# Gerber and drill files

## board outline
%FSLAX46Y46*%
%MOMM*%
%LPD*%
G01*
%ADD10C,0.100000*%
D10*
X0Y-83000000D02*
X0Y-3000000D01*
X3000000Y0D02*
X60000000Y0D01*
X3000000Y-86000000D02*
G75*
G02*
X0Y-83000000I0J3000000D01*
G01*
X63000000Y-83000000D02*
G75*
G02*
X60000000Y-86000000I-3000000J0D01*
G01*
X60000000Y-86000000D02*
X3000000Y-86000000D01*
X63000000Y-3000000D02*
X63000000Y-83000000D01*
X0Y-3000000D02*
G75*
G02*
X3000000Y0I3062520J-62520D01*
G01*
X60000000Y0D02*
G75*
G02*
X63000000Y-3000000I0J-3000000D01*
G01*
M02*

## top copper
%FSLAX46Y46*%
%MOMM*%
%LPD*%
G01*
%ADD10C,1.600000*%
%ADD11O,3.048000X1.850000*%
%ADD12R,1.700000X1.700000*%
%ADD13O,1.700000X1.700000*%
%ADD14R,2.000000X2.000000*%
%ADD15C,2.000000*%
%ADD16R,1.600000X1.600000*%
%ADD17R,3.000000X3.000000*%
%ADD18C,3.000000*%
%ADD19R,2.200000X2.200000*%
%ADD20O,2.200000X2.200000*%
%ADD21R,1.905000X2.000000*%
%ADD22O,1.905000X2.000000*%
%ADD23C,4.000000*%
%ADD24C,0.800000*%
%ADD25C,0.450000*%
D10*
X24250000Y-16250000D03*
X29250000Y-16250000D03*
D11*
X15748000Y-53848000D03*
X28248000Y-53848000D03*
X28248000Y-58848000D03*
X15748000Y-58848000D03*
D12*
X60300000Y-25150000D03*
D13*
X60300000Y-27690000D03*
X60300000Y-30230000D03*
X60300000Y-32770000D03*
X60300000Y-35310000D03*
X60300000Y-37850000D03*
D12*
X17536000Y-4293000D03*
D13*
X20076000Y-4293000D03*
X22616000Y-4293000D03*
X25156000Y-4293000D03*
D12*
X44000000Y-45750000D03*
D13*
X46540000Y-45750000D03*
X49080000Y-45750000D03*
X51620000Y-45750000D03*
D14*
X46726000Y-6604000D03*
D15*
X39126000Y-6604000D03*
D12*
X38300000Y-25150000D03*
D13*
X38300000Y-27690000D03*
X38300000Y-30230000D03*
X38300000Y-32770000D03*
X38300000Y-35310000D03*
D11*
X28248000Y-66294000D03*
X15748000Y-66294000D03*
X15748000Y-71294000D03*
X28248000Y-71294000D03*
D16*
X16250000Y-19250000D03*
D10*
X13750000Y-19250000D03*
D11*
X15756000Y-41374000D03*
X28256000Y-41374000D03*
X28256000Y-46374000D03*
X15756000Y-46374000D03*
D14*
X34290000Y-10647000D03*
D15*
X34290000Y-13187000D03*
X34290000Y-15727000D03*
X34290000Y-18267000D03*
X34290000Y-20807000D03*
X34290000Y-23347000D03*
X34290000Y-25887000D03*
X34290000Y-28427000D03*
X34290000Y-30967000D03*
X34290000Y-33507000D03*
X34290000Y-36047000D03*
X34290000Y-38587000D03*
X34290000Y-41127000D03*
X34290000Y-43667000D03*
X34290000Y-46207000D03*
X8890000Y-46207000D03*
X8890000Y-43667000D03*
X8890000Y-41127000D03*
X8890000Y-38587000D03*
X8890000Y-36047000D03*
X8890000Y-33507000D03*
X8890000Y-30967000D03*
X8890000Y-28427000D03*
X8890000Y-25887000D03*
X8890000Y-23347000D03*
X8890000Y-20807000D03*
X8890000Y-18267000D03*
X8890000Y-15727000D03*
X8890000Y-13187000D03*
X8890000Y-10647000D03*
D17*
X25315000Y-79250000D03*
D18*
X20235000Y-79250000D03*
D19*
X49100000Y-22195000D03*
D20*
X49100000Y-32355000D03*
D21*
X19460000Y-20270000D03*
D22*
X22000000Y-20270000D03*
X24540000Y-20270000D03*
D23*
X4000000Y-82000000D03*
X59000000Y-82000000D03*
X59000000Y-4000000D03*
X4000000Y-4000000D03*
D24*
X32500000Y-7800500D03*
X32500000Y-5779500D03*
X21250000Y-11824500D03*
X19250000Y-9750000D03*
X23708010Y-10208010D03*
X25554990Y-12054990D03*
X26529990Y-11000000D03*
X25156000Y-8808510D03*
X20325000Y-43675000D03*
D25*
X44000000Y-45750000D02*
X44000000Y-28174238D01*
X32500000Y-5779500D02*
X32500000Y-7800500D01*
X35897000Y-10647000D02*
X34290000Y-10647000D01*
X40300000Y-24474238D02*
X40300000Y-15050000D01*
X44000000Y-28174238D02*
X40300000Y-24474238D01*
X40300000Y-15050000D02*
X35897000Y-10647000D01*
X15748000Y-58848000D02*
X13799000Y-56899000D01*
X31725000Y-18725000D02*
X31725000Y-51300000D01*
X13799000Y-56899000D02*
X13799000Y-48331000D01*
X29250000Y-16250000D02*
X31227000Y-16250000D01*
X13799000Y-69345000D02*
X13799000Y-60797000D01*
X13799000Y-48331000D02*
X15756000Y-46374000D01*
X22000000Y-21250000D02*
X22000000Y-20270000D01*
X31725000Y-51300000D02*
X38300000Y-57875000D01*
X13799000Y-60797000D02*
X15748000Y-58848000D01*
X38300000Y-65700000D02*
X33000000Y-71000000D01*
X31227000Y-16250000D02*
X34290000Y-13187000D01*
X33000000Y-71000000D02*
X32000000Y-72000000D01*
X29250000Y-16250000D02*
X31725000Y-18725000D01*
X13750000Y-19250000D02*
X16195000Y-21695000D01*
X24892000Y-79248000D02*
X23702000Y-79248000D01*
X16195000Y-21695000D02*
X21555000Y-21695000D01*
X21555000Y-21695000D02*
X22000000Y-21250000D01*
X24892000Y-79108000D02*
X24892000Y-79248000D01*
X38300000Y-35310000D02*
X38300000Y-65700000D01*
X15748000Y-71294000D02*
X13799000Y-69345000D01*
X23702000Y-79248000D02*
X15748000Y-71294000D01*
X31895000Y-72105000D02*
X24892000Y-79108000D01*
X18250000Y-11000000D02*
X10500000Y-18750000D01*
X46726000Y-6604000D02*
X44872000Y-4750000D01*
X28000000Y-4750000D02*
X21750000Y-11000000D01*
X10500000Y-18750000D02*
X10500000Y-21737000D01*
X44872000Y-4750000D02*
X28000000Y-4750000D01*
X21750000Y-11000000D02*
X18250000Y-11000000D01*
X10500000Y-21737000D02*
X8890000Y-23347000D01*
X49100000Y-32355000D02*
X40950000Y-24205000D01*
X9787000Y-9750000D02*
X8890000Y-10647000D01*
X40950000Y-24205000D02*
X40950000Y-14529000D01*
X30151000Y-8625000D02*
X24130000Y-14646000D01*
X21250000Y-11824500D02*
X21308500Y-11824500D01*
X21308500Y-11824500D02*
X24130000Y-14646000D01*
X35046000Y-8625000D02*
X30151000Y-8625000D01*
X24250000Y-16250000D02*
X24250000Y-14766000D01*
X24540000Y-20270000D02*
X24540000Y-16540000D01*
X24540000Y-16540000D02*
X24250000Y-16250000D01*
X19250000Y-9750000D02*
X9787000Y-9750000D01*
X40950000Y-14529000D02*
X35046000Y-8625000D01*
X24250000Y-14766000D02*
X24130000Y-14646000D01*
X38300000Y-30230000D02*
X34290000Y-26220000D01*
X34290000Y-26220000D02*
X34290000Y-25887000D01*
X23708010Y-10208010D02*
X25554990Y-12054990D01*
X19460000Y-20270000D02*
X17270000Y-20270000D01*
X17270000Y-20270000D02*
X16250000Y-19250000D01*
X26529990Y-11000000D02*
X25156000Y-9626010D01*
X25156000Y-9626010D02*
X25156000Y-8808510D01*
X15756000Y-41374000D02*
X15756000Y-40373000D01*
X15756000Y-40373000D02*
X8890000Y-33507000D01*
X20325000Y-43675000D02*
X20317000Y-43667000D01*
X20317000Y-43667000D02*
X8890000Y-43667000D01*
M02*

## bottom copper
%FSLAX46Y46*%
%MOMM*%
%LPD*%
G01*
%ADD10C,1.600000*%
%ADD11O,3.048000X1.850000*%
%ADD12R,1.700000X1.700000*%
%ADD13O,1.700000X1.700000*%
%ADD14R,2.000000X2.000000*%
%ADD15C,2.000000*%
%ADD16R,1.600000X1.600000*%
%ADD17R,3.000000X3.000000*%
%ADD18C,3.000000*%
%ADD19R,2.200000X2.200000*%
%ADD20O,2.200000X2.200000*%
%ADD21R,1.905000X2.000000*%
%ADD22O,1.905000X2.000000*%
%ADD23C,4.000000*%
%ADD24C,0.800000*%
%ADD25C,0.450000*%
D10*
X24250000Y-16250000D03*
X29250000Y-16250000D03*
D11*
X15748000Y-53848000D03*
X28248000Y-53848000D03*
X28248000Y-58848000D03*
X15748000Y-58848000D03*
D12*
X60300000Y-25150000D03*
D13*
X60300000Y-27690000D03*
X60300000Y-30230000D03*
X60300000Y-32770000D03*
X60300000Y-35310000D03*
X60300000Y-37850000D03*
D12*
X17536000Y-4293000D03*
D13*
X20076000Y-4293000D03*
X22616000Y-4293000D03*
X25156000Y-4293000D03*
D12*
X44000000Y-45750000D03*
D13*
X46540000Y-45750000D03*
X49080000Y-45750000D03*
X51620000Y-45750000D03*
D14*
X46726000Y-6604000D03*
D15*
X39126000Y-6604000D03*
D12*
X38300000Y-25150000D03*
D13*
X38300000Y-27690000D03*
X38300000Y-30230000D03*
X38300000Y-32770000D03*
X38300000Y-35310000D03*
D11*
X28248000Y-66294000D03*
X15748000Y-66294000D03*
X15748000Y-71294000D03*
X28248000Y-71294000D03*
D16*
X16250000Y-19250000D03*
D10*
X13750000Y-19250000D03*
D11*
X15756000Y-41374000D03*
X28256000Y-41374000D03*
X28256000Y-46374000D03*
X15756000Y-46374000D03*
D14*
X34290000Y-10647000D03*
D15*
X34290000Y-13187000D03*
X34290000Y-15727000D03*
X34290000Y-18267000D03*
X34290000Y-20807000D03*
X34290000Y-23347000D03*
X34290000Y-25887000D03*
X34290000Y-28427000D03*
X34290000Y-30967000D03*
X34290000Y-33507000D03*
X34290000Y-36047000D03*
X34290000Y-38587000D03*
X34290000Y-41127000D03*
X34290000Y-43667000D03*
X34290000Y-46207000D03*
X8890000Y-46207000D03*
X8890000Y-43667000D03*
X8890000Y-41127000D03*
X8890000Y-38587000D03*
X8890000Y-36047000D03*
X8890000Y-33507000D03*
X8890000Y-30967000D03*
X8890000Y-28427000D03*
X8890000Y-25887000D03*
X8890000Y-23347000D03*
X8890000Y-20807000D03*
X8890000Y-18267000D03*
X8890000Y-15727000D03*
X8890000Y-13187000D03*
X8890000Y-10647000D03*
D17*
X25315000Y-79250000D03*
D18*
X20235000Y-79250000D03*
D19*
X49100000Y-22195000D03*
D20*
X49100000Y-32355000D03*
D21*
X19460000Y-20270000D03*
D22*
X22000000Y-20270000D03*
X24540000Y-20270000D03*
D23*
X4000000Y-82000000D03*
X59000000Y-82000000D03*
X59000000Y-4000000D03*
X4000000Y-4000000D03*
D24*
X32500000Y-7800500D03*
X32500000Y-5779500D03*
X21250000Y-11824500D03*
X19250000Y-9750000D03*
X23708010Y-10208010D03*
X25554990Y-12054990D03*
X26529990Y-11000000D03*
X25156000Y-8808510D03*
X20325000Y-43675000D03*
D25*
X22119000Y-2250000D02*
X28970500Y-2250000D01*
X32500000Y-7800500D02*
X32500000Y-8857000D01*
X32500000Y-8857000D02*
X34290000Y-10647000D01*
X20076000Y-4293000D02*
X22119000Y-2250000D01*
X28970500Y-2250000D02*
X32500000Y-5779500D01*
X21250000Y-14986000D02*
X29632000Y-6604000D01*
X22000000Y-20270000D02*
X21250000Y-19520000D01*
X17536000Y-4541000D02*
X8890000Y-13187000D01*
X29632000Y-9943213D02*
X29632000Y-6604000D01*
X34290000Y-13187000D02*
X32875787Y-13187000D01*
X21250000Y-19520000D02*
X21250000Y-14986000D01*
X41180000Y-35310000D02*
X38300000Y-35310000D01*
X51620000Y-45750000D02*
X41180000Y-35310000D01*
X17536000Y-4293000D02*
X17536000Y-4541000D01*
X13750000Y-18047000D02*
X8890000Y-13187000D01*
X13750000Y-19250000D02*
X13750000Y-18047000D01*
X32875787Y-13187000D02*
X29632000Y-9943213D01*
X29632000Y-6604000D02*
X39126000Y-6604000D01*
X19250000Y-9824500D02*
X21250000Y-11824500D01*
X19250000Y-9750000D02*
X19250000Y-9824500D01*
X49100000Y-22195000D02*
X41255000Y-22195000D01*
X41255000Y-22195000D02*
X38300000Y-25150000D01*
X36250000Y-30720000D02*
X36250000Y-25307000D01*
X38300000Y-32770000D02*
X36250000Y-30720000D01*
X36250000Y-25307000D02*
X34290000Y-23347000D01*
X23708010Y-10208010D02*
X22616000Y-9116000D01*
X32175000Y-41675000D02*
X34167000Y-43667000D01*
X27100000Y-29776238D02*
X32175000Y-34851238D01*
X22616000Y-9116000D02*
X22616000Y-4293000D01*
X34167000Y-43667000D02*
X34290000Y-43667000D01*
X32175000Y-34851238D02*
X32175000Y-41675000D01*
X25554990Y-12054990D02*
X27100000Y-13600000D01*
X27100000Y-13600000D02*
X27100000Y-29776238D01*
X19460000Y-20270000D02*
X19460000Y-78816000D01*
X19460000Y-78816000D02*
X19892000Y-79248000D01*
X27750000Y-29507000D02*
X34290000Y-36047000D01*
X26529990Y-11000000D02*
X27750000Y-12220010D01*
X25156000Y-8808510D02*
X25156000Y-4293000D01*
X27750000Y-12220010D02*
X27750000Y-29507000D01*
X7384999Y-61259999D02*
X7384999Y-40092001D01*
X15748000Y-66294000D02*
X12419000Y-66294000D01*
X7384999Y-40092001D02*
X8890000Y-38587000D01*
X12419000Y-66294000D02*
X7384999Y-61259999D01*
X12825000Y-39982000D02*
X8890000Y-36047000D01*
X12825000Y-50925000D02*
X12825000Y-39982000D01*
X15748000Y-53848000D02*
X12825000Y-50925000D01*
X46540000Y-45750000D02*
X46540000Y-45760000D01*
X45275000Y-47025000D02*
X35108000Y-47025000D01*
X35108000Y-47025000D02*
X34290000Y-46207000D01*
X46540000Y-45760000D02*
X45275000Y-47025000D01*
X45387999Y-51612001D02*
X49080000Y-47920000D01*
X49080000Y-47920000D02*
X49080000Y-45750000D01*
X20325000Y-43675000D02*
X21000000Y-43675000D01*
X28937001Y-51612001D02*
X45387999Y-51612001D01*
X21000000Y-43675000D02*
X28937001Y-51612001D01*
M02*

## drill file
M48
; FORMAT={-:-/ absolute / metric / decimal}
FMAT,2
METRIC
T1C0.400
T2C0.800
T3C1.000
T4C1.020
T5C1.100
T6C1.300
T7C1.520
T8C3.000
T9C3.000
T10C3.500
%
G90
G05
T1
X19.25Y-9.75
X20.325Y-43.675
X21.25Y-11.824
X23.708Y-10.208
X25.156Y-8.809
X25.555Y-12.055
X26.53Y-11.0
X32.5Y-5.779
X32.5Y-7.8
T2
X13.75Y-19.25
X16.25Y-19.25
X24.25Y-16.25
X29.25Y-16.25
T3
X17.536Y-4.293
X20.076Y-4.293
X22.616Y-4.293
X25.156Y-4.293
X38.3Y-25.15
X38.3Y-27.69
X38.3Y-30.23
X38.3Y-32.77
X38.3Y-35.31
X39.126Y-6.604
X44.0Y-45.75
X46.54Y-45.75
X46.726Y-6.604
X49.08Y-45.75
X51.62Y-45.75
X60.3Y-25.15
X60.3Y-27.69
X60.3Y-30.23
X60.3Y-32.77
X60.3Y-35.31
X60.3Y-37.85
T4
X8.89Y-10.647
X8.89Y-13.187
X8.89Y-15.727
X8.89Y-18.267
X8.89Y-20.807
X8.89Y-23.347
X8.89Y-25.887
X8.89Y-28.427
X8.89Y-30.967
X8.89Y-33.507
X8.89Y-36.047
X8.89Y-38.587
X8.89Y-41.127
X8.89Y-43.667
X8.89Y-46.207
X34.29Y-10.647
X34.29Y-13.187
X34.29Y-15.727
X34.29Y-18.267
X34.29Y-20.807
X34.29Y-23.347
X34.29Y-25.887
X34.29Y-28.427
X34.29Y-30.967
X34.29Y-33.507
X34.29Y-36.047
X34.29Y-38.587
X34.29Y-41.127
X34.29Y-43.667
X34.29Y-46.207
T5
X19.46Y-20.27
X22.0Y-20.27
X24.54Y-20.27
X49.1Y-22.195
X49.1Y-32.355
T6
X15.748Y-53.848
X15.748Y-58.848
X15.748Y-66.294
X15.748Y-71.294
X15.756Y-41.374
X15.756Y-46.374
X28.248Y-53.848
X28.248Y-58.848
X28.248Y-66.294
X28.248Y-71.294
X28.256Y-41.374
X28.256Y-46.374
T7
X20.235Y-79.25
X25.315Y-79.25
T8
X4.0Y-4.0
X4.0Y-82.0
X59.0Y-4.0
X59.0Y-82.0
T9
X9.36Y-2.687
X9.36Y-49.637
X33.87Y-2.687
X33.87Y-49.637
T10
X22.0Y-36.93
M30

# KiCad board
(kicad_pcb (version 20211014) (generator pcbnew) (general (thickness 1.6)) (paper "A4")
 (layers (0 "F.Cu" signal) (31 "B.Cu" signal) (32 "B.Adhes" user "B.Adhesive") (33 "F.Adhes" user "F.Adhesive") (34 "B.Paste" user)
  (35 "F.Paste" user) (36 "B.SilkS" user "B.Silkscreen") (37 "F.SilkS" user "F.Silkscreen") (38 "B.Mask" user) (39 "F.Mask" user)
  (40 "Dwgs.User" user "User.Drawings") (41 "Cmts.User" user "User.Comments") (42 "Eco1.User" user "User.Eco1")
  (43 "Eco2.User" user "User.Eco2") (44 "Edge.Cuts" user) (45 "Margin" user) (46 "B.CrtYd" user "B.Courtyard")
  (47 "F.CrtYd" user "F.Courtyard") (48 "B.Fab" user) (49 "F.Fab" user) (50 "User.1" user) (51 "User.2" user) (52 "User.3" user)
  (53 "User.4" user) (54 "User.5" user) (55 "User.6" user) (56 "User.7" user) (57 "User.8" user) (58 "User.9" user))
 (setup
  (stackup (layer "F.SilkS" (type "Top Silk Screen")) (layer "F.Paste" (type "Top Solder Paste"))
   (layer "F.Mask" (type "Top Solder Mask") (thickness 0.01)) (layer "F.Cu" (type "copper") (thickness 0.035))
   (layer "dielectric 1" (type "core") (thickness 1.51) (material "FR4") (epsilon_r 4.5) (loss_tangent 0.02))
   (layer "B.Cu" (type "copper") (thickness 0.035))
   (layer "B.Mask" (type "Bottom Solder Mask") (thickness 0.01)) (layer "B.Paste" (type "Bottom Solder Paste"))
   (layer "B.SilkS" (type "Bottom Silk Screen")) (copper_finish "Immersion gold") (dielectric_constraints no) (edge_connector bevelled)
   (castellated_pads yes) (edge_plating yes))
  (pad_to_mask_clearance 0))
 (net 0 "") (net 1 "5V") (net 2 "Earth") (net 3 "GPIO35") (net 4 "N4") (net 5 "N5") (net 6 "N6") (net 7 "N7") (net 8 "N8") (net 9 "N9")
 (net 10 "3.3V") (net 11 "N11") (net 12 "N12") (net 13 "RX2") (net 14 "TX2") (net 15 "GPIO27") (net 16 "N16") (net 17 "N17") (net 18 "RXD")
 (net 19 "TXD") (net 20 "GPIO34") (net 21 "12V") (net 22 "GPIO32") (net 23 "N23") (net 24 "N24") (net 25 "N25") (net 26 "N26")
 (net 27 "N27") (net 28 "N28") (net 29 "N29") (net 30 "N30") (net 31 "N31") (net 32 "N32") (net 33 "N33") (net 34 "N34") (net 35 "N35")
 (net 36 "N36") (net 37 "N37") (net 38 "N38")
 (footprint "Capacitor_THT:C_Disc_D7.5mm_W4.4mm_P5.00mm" (layer "F.Cu") (at 24.25 16.25)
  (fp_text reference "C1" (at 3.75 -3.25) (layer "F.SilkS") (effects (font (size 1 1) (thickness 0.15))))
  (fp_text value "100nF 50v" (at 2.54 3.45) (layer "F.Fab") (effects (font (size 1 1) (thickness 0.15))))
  (pad "1" thru_hole circle (at 0 0) (size 1.6 1.6) (drill 0.8) (layers *.Cu *.Mask) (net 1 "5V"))
  (pad "2" thru_hole circle (at 5 0) (size 1.6 1.6) (drill 0.8) (layers *.Cu *.Mask) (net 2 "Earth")))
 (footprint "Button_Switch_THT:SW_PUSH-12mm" (layer "F.Cu") (at 15.748 53.848)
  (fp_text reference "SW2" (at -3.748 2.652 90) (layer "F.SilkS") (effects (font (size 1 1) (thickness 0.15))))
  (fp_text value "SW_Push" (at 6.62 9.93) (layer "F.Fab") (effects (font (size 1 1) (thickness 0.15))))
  (pad "1" thru_hole oval (at 0 0) (size 3.048 1.85) (drill 1.3) (layers *.Cu *.Mask) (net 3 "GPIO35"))
  (pad "1" thru_hole oval (at 12.5 0) (size 3.048 1.85) (drill 1.3) (layers *.Cu *.Mask) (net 3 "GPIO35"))
  (pad "2" thru_hole oval (at 12.5 5) (size 3.048 1.85) (drill 1.3) (layers *.Cu *.Mask) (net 2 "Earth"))
  (pad "2" thru_hole oval (at 0 5) (size 3.048 1.85) (drill 1.3) (layers *.Cu *.Mask) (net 2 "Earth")))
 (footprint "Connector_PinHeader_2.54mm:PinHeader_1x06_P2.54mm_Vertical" (layer "F.Cu") (at 60.3 25.15)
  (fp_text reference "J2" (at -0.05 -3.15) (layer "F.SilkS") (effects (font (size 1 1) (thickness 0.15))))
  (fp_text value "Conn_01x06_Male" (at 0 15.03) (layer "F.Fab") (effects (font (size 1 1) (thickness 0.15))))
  (pad "1" thru_hole rect (at 0 0) (size 1.7 1.7) (drill 1) (layers *.Cu *.Mask) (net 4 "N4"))
  (pad "2" thru_hole oval (at 0 2.54) (size 1.7 1.7) (drill 1) (layers *.Cu *.Mask) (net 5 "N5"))
  (pad "3" thru_hole oval (at 0 5.08) (size 1.7 1.7) (drill 1) (layers *.Cu *.Mask) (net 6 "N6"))
  (pad "4" thru_hole oval (at 0 7.62) (size 1.7 1.7) (drill 1) (layers *.Cu *.Mask) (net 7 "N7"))
  (pad "5" thru_hole oval (at 0 10.16) (size 1.7 1.7) (drill 1) (layers *.Cu *.Mask) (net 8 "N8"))
  (pad "6" thru_hole oval (at 0 12.7) (size 1.7 1.7) (drill 1) (layers *.Cu *.Mask) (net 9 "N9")))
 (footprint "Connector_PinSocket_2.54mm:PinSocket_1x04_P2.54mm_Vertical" (layer "F.Cu") (at 17.536 4.293 90)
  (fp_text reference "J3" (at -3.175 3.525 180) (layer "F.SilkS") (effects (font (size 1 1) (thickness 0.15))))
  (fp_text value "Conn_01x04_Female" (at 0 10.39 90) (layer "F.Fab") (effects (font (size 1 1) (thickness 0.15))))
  (pad "1" thru_hole rect (at 0 0 90) (size 1.7 1.7) (drill 1) (layers *.Cu *.Mask) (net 2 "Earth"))
  (pad "2" thru_hole oval (at 0 2.54 90) (size 1.7 1.7) (drill 1) (layers *.Cu *.Mask) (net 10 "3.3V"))
  (pad "3" thru_hole oval (at 0 5.08 90) (size 1.7 1.7) (drill 1) (layers *.Cu *.Mask) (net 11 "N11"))
  (pad "4" thru_hole oval (at 0 7.62 90) (size 1.7 1.7) (drill 1) (layers *.Cu *.Mask) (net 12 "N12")))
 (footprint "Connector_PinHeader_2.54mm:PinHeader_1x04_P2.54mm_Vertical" (layer "F.Cu") (at 44 45.75 90)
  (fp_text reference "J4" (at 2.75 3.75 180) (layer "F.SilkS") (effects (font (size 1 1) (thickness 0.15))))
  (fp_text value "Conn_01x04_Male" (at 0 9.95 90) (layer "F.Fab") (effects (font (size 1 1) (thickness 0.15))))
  (pad "1" thru_hole rect (at 0 0 90) (size 1.7 1.7) (drill 1) (layers *.Cu *.Mask) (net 10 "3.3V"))
  (pad "2" thru_hole oval (at 0 2.54 90) (size 1.7 1.7) (drill 1) (layers *.Cu *.Mask) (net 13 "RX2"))
  (pad "3" thru_hole oval (at 0 5.08 90) (size 1.7 1.7) (drill 1) (layers *.Cu *.Mask) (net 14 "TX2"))
  (pad "4" thru_hole oval (at 0 7.62 90) (size 1.7 1.7) (drill 1) (layers *.Cu *.Mask) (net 2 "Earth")))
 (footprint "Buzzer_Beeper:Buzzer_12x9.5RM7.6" (layer "F.Cu") (at 46.726 6.604 180)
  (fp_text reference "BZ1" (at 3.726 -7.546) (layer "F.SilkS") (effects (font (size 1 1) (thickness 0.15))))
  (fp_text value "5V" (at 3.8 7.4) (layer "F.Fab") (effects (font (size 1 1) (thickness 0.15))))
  (pad "1" thru_hole rect (at 0 0 180) (size 2 2) (drill 1) (layers *.Cu *.Mask) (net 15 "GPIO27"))
  (pad "2" thru_hole circle (at 7.6 0 180) (size 2 2) (drill 1) (layers *.Cu *.Mask) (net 2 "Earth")))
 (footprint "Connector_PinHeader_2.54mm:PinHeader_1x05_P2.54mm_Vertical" (layer "F.Cu") (at 38.3 25.15)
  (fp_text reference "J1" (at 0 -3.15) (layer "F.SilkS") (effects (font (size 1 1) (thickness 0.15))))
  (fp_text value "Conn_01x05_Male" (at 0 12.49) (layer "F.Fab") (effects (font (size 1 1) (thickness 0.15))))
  (pad "1" thru_hole rect (at 0 0) (size 1.7 1.7) (drill 1) (layers *.Cu *.Mask) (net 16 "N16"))
  (pad "2" thru_hole oval (at 0 2.54) (size 1.7 1.7) (drill 1) (layers *.Cu *.Mask) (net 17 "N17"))
  (pad "3" thru_hole oval (at 0 5.08) (size 1.7 1.7) (drill 1) (layers *.Cu *.Mask) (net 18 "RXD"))
  (pad "4" thru_hole oval (at 0 7.62) (size 1.7 1.7) (drill 1) (layers *.Cu *.Mask) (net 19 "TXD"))
  (pad "5" thru_hole oval (at 0 10.16) (size 1.7 1.7) (drill 1) (layers *.Cu *.Mask) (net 2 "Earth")))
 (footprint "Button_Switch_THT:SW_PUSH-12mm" (layer "F.Cu") (at 15.748 66.294)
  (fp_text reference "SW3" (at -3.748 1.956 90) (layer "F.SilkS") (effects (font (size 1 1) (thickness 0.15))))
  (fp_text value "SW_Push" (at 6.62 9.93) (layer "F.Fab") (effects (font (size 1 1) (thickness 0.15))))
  (pad "1" thru_hole oval (at 12.5 0) (size 3.048 1.85) (drill 1.3) (layers *.Cu *.Mask) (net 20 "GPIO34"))
  (pad "1" thru_hole oval (at 0 0) (size 3.048 1.85) (drill 1.3) (layers *.Cu *.Mask) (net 20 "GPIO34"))
  (pad "2" thru_hole oval (at 0 5) (size 3.048 1.85) (drill 1.3) (layers *.Cu *.Mask) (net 2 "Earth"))
  (pad "2" thru_hole oval (at 12.5 5) (size 3.048 1.85) (drill 1.3) (layers *.Cu *.Mask) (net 2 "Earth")))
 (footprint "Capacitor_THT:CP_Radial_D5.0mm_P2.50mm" (layer "F.Cu") (at 16.25 19.25 180)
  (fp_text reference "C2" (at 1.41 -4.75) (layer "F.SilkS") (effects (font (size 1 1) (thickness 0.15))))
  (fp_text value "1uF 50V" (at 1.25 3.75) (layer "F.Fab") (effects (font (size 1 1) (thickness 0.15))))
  (pad "1" thru_hole rect (at 0 0 180) (size 1.6 1.6) (drill 0.8) (layers *.Cu *.Mask) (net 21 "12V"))
  (pad "2" thru_hole circle (at 2.5 0 180) (size 1.6 1.6) (drill 0.8) (layers *.Cu *.Mask) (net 2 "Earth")))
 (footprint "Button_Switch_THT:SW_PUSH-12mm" (layer "F.Cu") (at 15.756 41.374)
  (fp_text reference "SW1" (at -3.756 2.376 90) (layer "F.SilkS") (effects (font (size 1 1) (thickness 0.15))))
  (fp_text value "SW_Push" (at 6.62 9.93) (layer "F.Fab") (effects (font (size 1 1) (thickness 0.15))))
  (pad "1" thru_hole oval (at 0 0) (size 3.048 1.85) (drill 1.3) (layers *.Cu *.Mask) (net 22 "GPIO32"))
  (pad "1" thru_hole oval (at 12.5 0) (size 3.048 1.85) (drill 1.3) (layers *.Cu *.Mask) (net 22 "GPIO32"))
  (pad "2" thru_hole oval (at 12.5 5) (size 3.048 1.85) (drill 1.3) (layers *.Cu *.Mask) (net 2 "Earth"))
  (pad "2" thru_hole oval (at 0 5) (size 3.048 1.85) (drill 1.3) (layers *.Cu *.Mask) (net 2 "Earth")))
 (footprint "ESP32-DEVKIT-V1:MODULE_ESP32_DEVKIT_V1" (layer "B.Cu") (at 21.59 26.162 180)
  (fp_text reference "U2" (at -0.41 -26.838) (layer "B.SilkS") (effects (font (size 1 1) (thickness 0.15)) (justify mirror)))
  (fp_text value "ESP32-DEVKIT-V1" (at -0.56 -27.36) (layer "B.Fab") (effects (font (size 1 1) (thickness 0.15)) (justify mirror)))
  (pad "" np_thru_hole circle (at -12.28 -23.475 180) (size 3 3) (drill 3) (layers *.Cu *.Mask))
  (pad "" np_thru_hole circle (at 12.23 -23.475 180) (size 3 3) (drill 3) (layers *.Cu *.Mask))
  (pad "" np_thru_hole circle (at -12.28 23.475 180) (size 3 3) (drill 3) (layers *.Cu *.Mask))
  (pad "" np_thru_hole circle (at 12.23 23.475 180) (size 3 3) (drill 3) (layers *.Cu *.Mask))
  (pad "1" thru_hole rect (at -12.7 15.515 180) (size 2 2) (drill 1.02) (layers *.Cu *.Mask) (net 10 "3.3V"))
  (pad "2" thru_hole circle (at -12.7 12.975 180) (size 2 2) (drill 1.02) (layers *.Cu *.Mask) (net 2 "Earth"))
  (pad "3" thru_hole circle (at -12.7 10.435 180) (size 2 2) (drill 1.02) (layers *.Cu *.Mask) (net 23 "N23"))
  (pad "4" thru_hole circle (at -12.7 7.895 180) (size 2 2) (drill 1.02) (layers *.Cu *.Mask) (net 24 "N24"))
  (pad "5" thru_hole circle (at -12.7 5.355 180) (size 2 2) (drill 1.02) (layers *.Cu *.Mask) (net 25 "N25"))
  (pad "6" thru_hole circle (at -12.7 2.815 180) (size 2 2) (drill 1.02) (layers *.Cu *.Mask) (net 19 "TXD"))
  (pad "7" thru_hole circle (at -12.7 0.275 180) (size 2 2) (drill 1.02) (layers *.Cu *.Mask) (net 18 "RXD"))
  (pad "8" thru_hole circle (at -12.7 -2.265 180) (size 2 2) (drill 1.02) (layers *.Cu *.Mask) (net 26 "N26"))
  (pad "9" thru_hole circle (at -12.7 -4.805 180) (size 2 2) (drill 1.02) (layers *.Cu *.Mask) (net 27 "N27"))
  (pad "10" thru_hole circle (at -12.7 -7.345 180) (size 2 2) (drill 1.02) (layers *.Cu *.Mask) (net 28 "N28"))
  (pad "11" thru_hole circle (at -12.7 -9.885 180) (size 2 2) (drill 1.02) (layers *.Cu *.Mask) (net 12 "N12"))
  (pad "12" thru_hole circle (at -12.7 -12.425 180) (size 2 2) (drill 1.02) (layers *.Cu *.Mask) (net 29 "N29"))
  (pad "13" thru_hole circle (at -12.7 -14.965 180) (size 2 2) (drill 1.02) (layers *.Cu *.Mask) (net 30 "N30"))
  (pad "14" thru_hole circle (at -12.7 -17.505 180) (size 2 2) (drill 1.02) (layers *.Cu *.Mask) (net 11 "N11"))
  (pad "15" thru_hole circle (at -12.7 -20.045 180) (size 2 2) (drill 1.02) (layers *.Cu *.Mask) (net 13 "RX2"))
  (pad "16" thru_hole circle (at 12.7 -20.045 180) (size 2 2) (drill 1.02) (layers *.Cu *.Mask) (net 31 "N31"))
  (pad "17" thru_hole circle (at 12.7 -17.505 180) (size 2 2) (drill 1.02) (layers *.Cu *.Mask) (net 14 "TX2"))
  (pad "18" thru_hole circle (at 12.7 -14.965 180) (size 2 2) (drill 1.02) (layers *.Cu *.Mask) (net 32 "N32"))
  (pad "19" thru_hole circle (at 12.7 -12.425 180) (size 2 2) (drill 1.02) (layers *.Cu *.Mask) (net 20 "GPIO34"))
  (pad "20" thru_hole circle (at 12.7 -9.885 180) (size 2 2) (drill 1.02) (layers *.Cu *.Mask) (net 3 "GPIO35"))
  (pad "21" thru_hole circle (at 12.7 -7.345 180) (size 2 2) (drill 1.02) (layers *.Cu *.Mask) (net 22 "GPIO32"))
  (pad "22" thru_hole circle (at 12.7 -4.805 180) (size 2 2) (drill 1.02) (layers *.Cu *.Mask) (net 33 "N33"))
  (pad "23" thru_hole circle (at 12.7 -2.265 180) (size 2 2) (drill 1.02) (layers *.Cu *.Mask) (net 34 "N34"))
  (pad "24" thru_hole circle (at 12.7 0.275 180) (size 2 2) (drill 1.02) (layers *.Cu *.Mask) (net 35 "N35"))
  (pad "25" thru_hole circle (at 12.7 2.815 180) (size 2 2) (drill 1.02) (layers *.Cu *.Mask) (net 15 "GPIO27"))
  (pad "26" thru_hole circle (at 12.7 5.355 180) (size 2 2) (drill 1.02) (layers *.Cu *.Mask) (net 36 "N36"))
  (pad "27" thru_hole circle (at 12.7 7.895 180) (size 2 2) (drill 1.02) (layers *.Cu *.Mask) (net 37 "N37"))
  (pad "28" thru_hole circle (at 12.7 10.435 180) (size 2 2) (drill 1.02) (layers *.Cu *.Mask) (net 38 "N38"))
  (pad "29" thru_hole circle (at 12.7 12.975 180) (size 2 2) (drill 1.02) (layers *.Cu *.Mask) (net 2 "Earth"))
  (pad "30" thru_hole circle (at 12.7 15.515 180) (size 2 2) (drill 1.02) (layers *.Cu *.Mask) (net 1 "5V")))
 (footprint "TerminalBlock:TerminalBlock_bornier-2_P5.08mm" (layer "B.Cu") (at 25.315 79.25 180)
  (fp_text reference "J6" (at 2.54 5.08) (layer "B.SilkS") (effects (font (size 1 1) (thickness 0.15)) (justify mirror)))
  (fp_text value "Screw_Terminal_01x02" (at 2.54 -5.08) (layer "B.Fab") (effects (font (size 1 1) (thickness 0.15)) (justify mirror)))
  (pad "1" thru_hole rect (at 0 0 180) (size 3 3) (drill 1.52) (layers *.Cu *.Mask) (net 2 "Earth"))
  (pad "2" thru_hole circle (at 5.08 0 180) (size 3 3) (drill 1.52) (layers *.Cu *.Mask) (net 21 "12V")))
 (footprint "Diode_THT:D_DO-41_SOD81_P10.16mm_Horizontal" (layer "B.Cu") (at 49.1 22.195 -90)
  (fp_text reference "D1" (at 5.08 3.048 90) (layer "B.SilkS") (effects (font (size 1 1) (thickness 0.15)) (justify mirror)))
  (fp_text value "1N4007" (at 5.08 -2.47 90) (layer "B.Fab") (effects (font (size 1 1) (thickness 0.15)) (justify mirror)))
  (pad "1" thru_hole rect (at 0 0 270) (size 2.2 2.2) (drill 1.1) (layers *.Cu *.Mask) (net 16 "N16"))
  (pad "2" thru_hole oval (at 10.16 0 270) (size 2.2 2.2) (drill 1.1) (layers *.Cu *.Mask) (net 1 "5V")))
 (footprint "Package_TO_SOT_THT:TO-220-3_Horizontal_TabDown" (layer "B.Cu") (at 19.46 20.27)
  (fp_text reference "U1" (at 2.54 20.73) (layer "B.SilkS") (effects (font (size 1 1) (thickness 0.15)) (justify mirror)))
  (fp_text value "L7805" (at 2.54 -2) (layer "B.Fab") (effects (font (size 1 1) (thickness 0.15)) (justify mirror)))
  (pad "" np_thru_hole oval (at 2.54 16.66) (size 3.5 3.5) (drill 3.5) (layers *.Cu *.Mask))
  (pad "1" thru_hole rect (at 0 0) (size 1.905 2) (drill 1.1) (layers *.Cu *.Mask) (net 21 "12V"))
  (pad "2" thru_hole oval (at 2.54 0) (size 1.905 2) (drill 1.1) (layers *.Cu *.Mask) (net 2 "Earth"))
  (pad "3" thru_hole oval (at 5.08 0) (size 1.905 2) (drill 1.1) (layers *.Cu *.Mask) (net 1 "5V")))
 (gr_line (start 0 83) (end 0 3) (layer "Edge.Cuts") (width 0.1))
 (gr_line (start 3 0) (end 60 0) (layer "Edge.Cuts") (width 0.1))
 (gr_arc (start 3 86) (mid 0.87868 85.12132) (end 0 83) (layer "Edge.Cuts") (width 0.1))
 (gr_arc (start 63 83) (mid 62.12132 85.12132) (end 60 86) (layer "Edge.Cuts") (width 0.1))
 (gr_line (start 60 86) (end 3 86) (layer "Edge.Cuts") (width 0.1))
 (gr_line (start 63 3) (end 63 83) (layer "Edge.Cuts") (width 0.1))
 (gr_arc (start 0 3) (mid 0.89654 0.89654) (end 3 0) (layer "Edge.Cuts") (width 0.1))
 (gr_arc (start 60 0) (mid 62.12132 0.87868) (end 63 3) (layer "Edge.Cuts") (width 0.1))
 (via (at 4 82) (size 4) (drill 3) (layers "F.Cu" "B.Cu") (free) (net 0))
 (via (at 59 82) (size 4) (drill 3) (layers "F.Cu" "B.Cu") (free) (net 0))
 (via (at 59 4) (size 4) (drill 3) (layers "F.Cu" "B.Cu") (free) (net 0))
 (via locked (at 4 4) (size 4) (drill 3) (layers "F.Cu" "B.Cu") (free) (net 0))
 (segment (start 44 45.75) (end 44 28.174238) (width 0.45) (layer "F.Cu") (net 10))
 (segment (start 32.5 5.7795) (end 32.5 7.8005) (width 0.45) (layer "F.Cu") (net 10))
 (segment (start 35.897 10.647) (end 34.29 10.647) (width 0.45) (layer "F.Cu") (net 10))
 (segment (start 40.3 24.474238) (end 40.3 15.05) (width 0.45) (layer "F.Cu") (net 10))
 (segment (start 44 28.174238) (end 40.3 24.474238) (width 0.45) (layer "F.Cu") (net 10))
 (segment (start 40.3 15.05) (end 35.897 10.647) (width 0.45) (layer "F.Cu") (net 10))
 (via (at 32.5 7.8005) (size 0.8) (drill 0.4) (layers "F.Cu" "B.Cu") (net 10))
 (via (at 32.5 5.7795) (size 0.8) (drill 0.4) (layers "F.Cu" "B.Cu") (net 10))
 (segment (start 22.119 2.25) (end 28.9705 2.25) (width 0.45) (layer "B.Cu") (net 10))
 (segment (start 32.5 7.8005) (end 32.5 8.857) (width 0.45) (layer "B.Cu") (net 10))
 (segment (start 32.5 8.857) (end 34.29 10.647) (width 0.45) (layer "B.Cu") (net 10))
 (segment (start 20.076 4.293) (end 22.119 2.25) (width 0.45) (layer "B.Cu") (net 10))
 (segment (start 28.9705 2.25) (end 32.5 5.7795) (width 0.45) (layer "B.Cu") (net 10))
 (segment (start 15.748 58.848) (end 13.799 56.899) (width 0.45) (layer "F.Cu") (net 2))
 (segment (start 31.725 18.725) (end 31.725 51.3) (width 0.45) (layer "F.Cu") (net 2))
 (segment (start 13.799 56.899) (end 13.799 48.331) (width 0.45) (layer "F.Cu") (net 2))
 (segment (start 29.25 16.25) (end 31.227 16.25) (width 0.45) (layer "F.Cu") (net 2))
 (segment (start 13.799 69.345) (end 13.799 60.797) (width 0.45) (layer "F.Cu") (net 2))
 (segment (start 13.799 48.331) (end 15.756 46.374) (width 0.45) (layer "F.Cu") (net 2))
 (segment (start 22 21.25) (end 22 20.27) (width 0.45) (layer "F.Cu") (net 2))
 (segment (start 31.725 51.3) (end 38.3 57.875) (width 0.45) (layer "F.Cu") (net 2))
 (segment (start 13.799 60.797) (end 15.748 58.848) (width 0.45) (layer "F.Cu") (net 2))
 (segment (start 38.3 65.7) (end 33 71) (width 0.45) (layer "F.Cu") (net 2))
 (segment (start 31.227 16.25) (end 34.29 13.187) (width 0.45) (layer "F.Cu") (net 2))
 (segment (start 33 71) (end 32 72) (width 0.45) (layer "F.Cu") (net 2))
 (segment (start 29.25 16.25) (end 31.725 18.725) (width 0.45) (layer "F.Cu") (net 2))
 (segment (start 13.75 19.25) (end 16.195 21.695) (width 0.45) (layer "F.Cu") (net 2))
 (segment (start 24.892 79.248) (end 23.702 79.248) (width 0.45) (layer "F.Cu") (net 2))
 (segment (start 16.195 21.695) (end 21.555 21.695) (width 0.45) (layer "F.Cu") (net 2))
 (segment (start 21.555 21.695) (end 22 21.25) (width 0.45) (layer "F.Cu") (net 2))
 (segment (start 24.892 79.108) (end 24.892 79.248) (width 0.45) (layer "F.Cu") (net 2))
 (segment (start 38.3 35.31) (end 38.3 65.7) (width 0.45) (layer "F.Cu") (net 2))
 (segment (start 15.748 71.294) (end 13.799 69.345) (width 0.45) (layer "F.Cu") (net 2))
 (segment (start 23.702 79.248) (end 15.748 71.294) (width 0.45) (layer "F.Cu") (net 2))
 (segment (start 31.895 72.105) (end 24.892 79.108) (width 0.45) (layer "F.Cu") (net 2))
 (segment (start 21.25 14.986) (end 29.632 6.604) (width 0.45) (layer "B.Cu") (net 2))
 (segment (start 22 20.27) (end 21.25 19.52) (width 0.45) (layer "B.Cu") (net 2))
 (segment (start 17.536 4.541) (end 8.89 13.187) (width 0.45) (layer "B.Cu") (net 2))
 (segment (start 29.632 9.943213) (end 29.632 6.604) (width 0.45) (layer "B.Cu") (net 2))
 (segment (start 34.29 13.187) (end 32.875787 13.187) (width 0.45) (layer "B.Cu") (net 2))
 (segment (start 21.25 19.52) (end 21.25 14.986) (width 0.45) (layer "B.Cu") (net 2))
 (segment (start 41.18 35.31) (end 38.3 35.31) (width 0.45) (layer "B.Cu") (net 2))
 (segment (start 51.62 45.75) (end 41.18 35.31) (width 0.45) (layer "B.Cu") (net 2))
 (segment (start 17.536 4.293) (end 17.536 4.541) (width 0.45) (layer "B.Cu") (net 2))
 (segment (start 13.75 18.047) (end 8.89 13.187) (width 0.45) (layer "B.Cu") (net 2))
 (segment (start 13.75 19.25) (end 13.75 18.047) (width 0.45) (layer "B.Cu") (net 2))
 (segment (start 32.875787 13.187) (end 29.632 9.943213) (width 0.45) (layer "B.Cu") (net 2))
 (segment (start 29.632 6.604) (end 39.126 6.604) (width 0.45) (layer "B.Cu") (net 2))
 (segment (start 18.25 11) (end 10.5 18.75) (width 0.45) (layer "F.Cu") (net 15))
 (segment (start 46.726 6.604) (end 44.872 4.75) (width 0.45) (layer "F.Cu") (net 15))
 (segment (start 28 4.75) (end 21.75 11) (width 0.45) (layer "F.Cu") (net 15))
 (segment (start 10.5 18.75) (end 10.5 21.737) (width 0.45) (layer "F.Cu") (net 15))
 (segment (start 44.872 4.75) (end 28 4.75) (width 0.45) (layer "F.Cu") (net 15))
 (segment (start 21.75 11) (end 18.25 11) (width 0.45) (layer "F.Cu") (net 15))
 (segment (start 10.5 21.737) (end 8.89 23.347) (width 0.45) (layer "F.Cu") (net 15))
 (segment (start 49.1 32.355) (end 40.95 24.205) (width 0.45) (layer "F.Cu") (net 1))
 (segment (start 9.787 9.75) (end 8.89 10.647) (width 0.45) (layer "F.Cu") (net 1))
 (segment (start 40.95 24.205) (end 40.95 14.529) (width 0.45) (layer "F.Cu") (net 1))
 (segment (start 30.151 8.625) (end 24.13 14.646) (width 0.45) (layer "F.Cu") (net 1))
 (segment (start 21.25 11.8245) (end 21.3085 11.8245) (width 0.45) (layer "F.Cu") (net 1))
 (segment (start 21.3085 11.8245) (end 24.13 14.646) (width 0.45) (layer "F.Cu") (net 1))
 (segment (start 35.046 8.625) (end 30.151 8.625) (width 0.45) (layer "F.Cu") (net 1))
 (segment (start 24.25 16.25) (end 24.25 14.766) (width 0.45) (layer "F.Cu") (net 1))
 (segment (start 24.54 20.27) (end 24.54 16.54) (width 0.45) (layer "F.Cu") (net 1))
 (segment (start 24.54 16.54) (end 24.25 16.25) (width 0.45) (layer "F.Cu") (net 1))
 (segment (start 19.25 9.75) (end 9.787 9.75) (width 0.45) (layer "F.Cu") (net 1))
 (segment (start 40.95 14.529) (end 35.046 8.625) (width 0.45) (layer "F.Cu") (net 1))
 (segment (start 24.25 14.766) (end 24.13 14.646) (width 0.45) (layer "F.Cu") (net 1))
 (via (at 21.25 11.8245) (size 0.8) (drill 0.4) (layers "F.Cu" "B.Cu") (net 1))
 (via (at 19.25 9.75) (size 0.8) (drill 0.4) (layers "F.Cu" "B.Cu") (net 1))
 (segment (start 19.25 9.8245) (end 21.25 11.8245) (width 0.45) (layer "B.Cu") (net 1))
 (segment (start 19.25 9.75) (end 19.25 9.8245) (width 0.45) (layer "B.Cu") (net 1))
 (segment (start 49.1 22.195) (end 41.255 22.195) (width 0.45) (layer "B.Cu") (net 16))
 (segment (start 41.255 22.195) (end 38.3 25.15) (width 0.45) (layer "B.Cu") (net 16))
 (segment (start 38.3 30.23) (end 34.29 26.22) (width 0.45) (layer "F.Cu") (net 18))
 (segment (start 34.29 26.22) (end 34.29 25.887) (width 0.45) (layer "F.Cu") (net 18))
 (segment (start 36.25 30.72) (end 36.25 25.307) (width 0.45) (layer "B.Cu") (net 19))
 (segment (start 38.3 32.77) (end 36.25 30.72) (width 0.45) (layer "B.Cu") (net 19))
 (segment (start 36.25 25.307) (end 34.29 23.347) (width 0.45) (layer "B.Cu") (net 19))
 (segment (start 23.70801 10.20801) (end 25.55499 12.05499) (width 0.45) (layer "F.Cu") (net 11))
 (via (at 23.70801 10.20801) (size 0.8) (drill 0.4) (layers "F.Cu" "B.Cu") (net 11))
 (via (at 25.55499 12.05499) (size 0.8) (drill 0.4) (layers "F.Cu" "B.Cu") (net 11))
 (segment (start 23.70801 10.20801) (end 22.616 9.116) (width 0.45) (layer "B.Cu") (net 11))
 (segment (start 32.175 41.675) (end 34.167 43.667) (width 0.45) (layer "B.Cu") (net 11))
 (segment (start 27.1 29.776238) (end 32.175 34.851238) (width 0.45) (layer "B.Cu") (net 11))
 (segment (start 22.616 9.116) (end 22.616 4.293) (width 0.45) (layer "B.Cu") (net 11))
 (segment (start 34.167 43.667) (end 34.29 43.667) (width 0.45) (layer "B.Cu") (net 11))
 (segment (start 32.175 34.851238) (end 32.175 41.675) (width 0.45) (layer "B.Cu") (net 11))
 (segment (start 25.55499 12.05499) (end 27.1 13.6) (width 0.45) (layer "B.Cu") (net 11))
 (segment (start 27.1 13.6) (end 27.1 29.776238) (width 0.45) (layer "B.Cu") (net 11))
 (segment (start 19.46 20.27) (end 17.27 20.27) (width 0.45) (layer "F.Cu") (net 21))
 (segment (start 17.27 20.27) (end 16.25 19.25) (width 0.45) (layer "F.Cu") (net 21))
 (segment (start 19.46 20.27) (end 19.46 78.816) (width 0.45) (layer "B.Cu") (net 21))
 (segment (start 19.46 78.816) (end 19.892 79.248) (width 0.45) (layer "B.Cu") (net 21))
 (segment (start 26.52999 11) (end 25.156 9.62601) (width 0.45) (layer "F.Cu") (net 12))
 (segment (start 25.156 9.62601) (end 25.156 8.80851) (width 0.45) (layer "F.Cu") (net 12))
 (via (at 26.52999 11) (size 0.8) (drill 0.4) (layers "F.Cu" "B.Cu") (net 12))
 (via (at 25.156 8.80851) (size 0.8) (drill 0.4) (layers "F.Cu" "B.Cu") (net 12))
 (segment (start 27.75 29.507) (end 34.29 36.047) (width 0.45) (layer "B.Cu") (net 12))
 (segment (start 26.52999 11) (end 27.75 12.22001) (width 0.45) (layer "B.Cu") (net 12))
 (segment (start 25.156 8.80851) (end 25.156 4.293) (width 0.45) (layer "B.Cu") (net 12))
 (segment (start 27.75 12.22001) (end 27.75 29.507) (width 0.45) (layer "B.Cu") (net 12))
 (segment (start 7.384999 61.259999) (end 7.384999 40.092001) (width 0.45) (layer "B.Cu") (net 20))
 (segment (start 15.748 66.294) (end 12.419 66.294) (width 0.45) (layer "B.Cu") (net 20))
 (segment (start 7.384999 40.092001) (end 8.89 38.587) (width 0.45) (layer "B.Cu") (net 20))
 (segment (start 12.419 66.294) (end 7.384999 61.259999) (width 0.45) (layer "B.Cu") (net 20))
 (segment (start 12.825 39.982) (end 8.89 36.047) (width 0.45) (layer "B.Cu") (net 3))
 (segment (start 12.825 50.925) (end 12.825 39.982) (width 0.45) (layer "B.Cu") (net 3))
 (segment (start 15.748 53.848) (end 12.825 50.925) (width 0.45) (layer "B.Cu") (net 3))
 (segment (start 15.756 41.374) (end 15.756 40.373) (width 0.45) (layer "F.Cu") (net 22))
 (segment (start 15.756 40.373) (end 8.89 33.507) (width 0.45) (layer "F.Cu") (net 22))
 (segment (start 46.54 45.75) (end 46.54 45.76) (width 0.45) (layer "B.Cu") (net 13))
 (segment (start 45.275 47.025) (end 35.108 47.025) (width 0.45) (layer "B.Cu") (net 13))
 (segment (start 35.108 47.025) (end 34.29 46.207) (width 0.45) (layer "B.Cu") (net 13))
 (segment (start 46.54 45.76) (end 45.275 47.025) (width 0.45) (layer "B.Cu") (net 13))
 (segment (start 20.325 43.675) (end 20.317 43.667) (width 0.45) (layer "F.Cu") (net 14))
 (segment (start 20.317 43.667) (end 8.89 43.667) (width 0.45) (layer "F.Cu") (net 14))
 (via (at 20.325 43.675) (size 0.8) (drill 0.4) (layers "F.Cu" "B.Cu") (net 14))
 (segment (start 45.387999 51.612001) (end 49.08 47.92) (width 0.45) (layer "B.Cu") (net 14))
 (segment (start 49.08 47.92) (end 49.08 45.75) (width 0.45) (layer "B.Cu") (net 14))
 (segment (start 20.325 43.675) (end 21 43.675) (width 0.45) (layer "B.Cu") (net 14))
 (segment (start 28.937001 51.612001) (end 45.387999 51.612001) (width 0.45) (layer "B.Cu") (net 14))
 (segment (start 21 43.675) (end 28.937001 51.612001) (width 0.45) (layer "B.Cu") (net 14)))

